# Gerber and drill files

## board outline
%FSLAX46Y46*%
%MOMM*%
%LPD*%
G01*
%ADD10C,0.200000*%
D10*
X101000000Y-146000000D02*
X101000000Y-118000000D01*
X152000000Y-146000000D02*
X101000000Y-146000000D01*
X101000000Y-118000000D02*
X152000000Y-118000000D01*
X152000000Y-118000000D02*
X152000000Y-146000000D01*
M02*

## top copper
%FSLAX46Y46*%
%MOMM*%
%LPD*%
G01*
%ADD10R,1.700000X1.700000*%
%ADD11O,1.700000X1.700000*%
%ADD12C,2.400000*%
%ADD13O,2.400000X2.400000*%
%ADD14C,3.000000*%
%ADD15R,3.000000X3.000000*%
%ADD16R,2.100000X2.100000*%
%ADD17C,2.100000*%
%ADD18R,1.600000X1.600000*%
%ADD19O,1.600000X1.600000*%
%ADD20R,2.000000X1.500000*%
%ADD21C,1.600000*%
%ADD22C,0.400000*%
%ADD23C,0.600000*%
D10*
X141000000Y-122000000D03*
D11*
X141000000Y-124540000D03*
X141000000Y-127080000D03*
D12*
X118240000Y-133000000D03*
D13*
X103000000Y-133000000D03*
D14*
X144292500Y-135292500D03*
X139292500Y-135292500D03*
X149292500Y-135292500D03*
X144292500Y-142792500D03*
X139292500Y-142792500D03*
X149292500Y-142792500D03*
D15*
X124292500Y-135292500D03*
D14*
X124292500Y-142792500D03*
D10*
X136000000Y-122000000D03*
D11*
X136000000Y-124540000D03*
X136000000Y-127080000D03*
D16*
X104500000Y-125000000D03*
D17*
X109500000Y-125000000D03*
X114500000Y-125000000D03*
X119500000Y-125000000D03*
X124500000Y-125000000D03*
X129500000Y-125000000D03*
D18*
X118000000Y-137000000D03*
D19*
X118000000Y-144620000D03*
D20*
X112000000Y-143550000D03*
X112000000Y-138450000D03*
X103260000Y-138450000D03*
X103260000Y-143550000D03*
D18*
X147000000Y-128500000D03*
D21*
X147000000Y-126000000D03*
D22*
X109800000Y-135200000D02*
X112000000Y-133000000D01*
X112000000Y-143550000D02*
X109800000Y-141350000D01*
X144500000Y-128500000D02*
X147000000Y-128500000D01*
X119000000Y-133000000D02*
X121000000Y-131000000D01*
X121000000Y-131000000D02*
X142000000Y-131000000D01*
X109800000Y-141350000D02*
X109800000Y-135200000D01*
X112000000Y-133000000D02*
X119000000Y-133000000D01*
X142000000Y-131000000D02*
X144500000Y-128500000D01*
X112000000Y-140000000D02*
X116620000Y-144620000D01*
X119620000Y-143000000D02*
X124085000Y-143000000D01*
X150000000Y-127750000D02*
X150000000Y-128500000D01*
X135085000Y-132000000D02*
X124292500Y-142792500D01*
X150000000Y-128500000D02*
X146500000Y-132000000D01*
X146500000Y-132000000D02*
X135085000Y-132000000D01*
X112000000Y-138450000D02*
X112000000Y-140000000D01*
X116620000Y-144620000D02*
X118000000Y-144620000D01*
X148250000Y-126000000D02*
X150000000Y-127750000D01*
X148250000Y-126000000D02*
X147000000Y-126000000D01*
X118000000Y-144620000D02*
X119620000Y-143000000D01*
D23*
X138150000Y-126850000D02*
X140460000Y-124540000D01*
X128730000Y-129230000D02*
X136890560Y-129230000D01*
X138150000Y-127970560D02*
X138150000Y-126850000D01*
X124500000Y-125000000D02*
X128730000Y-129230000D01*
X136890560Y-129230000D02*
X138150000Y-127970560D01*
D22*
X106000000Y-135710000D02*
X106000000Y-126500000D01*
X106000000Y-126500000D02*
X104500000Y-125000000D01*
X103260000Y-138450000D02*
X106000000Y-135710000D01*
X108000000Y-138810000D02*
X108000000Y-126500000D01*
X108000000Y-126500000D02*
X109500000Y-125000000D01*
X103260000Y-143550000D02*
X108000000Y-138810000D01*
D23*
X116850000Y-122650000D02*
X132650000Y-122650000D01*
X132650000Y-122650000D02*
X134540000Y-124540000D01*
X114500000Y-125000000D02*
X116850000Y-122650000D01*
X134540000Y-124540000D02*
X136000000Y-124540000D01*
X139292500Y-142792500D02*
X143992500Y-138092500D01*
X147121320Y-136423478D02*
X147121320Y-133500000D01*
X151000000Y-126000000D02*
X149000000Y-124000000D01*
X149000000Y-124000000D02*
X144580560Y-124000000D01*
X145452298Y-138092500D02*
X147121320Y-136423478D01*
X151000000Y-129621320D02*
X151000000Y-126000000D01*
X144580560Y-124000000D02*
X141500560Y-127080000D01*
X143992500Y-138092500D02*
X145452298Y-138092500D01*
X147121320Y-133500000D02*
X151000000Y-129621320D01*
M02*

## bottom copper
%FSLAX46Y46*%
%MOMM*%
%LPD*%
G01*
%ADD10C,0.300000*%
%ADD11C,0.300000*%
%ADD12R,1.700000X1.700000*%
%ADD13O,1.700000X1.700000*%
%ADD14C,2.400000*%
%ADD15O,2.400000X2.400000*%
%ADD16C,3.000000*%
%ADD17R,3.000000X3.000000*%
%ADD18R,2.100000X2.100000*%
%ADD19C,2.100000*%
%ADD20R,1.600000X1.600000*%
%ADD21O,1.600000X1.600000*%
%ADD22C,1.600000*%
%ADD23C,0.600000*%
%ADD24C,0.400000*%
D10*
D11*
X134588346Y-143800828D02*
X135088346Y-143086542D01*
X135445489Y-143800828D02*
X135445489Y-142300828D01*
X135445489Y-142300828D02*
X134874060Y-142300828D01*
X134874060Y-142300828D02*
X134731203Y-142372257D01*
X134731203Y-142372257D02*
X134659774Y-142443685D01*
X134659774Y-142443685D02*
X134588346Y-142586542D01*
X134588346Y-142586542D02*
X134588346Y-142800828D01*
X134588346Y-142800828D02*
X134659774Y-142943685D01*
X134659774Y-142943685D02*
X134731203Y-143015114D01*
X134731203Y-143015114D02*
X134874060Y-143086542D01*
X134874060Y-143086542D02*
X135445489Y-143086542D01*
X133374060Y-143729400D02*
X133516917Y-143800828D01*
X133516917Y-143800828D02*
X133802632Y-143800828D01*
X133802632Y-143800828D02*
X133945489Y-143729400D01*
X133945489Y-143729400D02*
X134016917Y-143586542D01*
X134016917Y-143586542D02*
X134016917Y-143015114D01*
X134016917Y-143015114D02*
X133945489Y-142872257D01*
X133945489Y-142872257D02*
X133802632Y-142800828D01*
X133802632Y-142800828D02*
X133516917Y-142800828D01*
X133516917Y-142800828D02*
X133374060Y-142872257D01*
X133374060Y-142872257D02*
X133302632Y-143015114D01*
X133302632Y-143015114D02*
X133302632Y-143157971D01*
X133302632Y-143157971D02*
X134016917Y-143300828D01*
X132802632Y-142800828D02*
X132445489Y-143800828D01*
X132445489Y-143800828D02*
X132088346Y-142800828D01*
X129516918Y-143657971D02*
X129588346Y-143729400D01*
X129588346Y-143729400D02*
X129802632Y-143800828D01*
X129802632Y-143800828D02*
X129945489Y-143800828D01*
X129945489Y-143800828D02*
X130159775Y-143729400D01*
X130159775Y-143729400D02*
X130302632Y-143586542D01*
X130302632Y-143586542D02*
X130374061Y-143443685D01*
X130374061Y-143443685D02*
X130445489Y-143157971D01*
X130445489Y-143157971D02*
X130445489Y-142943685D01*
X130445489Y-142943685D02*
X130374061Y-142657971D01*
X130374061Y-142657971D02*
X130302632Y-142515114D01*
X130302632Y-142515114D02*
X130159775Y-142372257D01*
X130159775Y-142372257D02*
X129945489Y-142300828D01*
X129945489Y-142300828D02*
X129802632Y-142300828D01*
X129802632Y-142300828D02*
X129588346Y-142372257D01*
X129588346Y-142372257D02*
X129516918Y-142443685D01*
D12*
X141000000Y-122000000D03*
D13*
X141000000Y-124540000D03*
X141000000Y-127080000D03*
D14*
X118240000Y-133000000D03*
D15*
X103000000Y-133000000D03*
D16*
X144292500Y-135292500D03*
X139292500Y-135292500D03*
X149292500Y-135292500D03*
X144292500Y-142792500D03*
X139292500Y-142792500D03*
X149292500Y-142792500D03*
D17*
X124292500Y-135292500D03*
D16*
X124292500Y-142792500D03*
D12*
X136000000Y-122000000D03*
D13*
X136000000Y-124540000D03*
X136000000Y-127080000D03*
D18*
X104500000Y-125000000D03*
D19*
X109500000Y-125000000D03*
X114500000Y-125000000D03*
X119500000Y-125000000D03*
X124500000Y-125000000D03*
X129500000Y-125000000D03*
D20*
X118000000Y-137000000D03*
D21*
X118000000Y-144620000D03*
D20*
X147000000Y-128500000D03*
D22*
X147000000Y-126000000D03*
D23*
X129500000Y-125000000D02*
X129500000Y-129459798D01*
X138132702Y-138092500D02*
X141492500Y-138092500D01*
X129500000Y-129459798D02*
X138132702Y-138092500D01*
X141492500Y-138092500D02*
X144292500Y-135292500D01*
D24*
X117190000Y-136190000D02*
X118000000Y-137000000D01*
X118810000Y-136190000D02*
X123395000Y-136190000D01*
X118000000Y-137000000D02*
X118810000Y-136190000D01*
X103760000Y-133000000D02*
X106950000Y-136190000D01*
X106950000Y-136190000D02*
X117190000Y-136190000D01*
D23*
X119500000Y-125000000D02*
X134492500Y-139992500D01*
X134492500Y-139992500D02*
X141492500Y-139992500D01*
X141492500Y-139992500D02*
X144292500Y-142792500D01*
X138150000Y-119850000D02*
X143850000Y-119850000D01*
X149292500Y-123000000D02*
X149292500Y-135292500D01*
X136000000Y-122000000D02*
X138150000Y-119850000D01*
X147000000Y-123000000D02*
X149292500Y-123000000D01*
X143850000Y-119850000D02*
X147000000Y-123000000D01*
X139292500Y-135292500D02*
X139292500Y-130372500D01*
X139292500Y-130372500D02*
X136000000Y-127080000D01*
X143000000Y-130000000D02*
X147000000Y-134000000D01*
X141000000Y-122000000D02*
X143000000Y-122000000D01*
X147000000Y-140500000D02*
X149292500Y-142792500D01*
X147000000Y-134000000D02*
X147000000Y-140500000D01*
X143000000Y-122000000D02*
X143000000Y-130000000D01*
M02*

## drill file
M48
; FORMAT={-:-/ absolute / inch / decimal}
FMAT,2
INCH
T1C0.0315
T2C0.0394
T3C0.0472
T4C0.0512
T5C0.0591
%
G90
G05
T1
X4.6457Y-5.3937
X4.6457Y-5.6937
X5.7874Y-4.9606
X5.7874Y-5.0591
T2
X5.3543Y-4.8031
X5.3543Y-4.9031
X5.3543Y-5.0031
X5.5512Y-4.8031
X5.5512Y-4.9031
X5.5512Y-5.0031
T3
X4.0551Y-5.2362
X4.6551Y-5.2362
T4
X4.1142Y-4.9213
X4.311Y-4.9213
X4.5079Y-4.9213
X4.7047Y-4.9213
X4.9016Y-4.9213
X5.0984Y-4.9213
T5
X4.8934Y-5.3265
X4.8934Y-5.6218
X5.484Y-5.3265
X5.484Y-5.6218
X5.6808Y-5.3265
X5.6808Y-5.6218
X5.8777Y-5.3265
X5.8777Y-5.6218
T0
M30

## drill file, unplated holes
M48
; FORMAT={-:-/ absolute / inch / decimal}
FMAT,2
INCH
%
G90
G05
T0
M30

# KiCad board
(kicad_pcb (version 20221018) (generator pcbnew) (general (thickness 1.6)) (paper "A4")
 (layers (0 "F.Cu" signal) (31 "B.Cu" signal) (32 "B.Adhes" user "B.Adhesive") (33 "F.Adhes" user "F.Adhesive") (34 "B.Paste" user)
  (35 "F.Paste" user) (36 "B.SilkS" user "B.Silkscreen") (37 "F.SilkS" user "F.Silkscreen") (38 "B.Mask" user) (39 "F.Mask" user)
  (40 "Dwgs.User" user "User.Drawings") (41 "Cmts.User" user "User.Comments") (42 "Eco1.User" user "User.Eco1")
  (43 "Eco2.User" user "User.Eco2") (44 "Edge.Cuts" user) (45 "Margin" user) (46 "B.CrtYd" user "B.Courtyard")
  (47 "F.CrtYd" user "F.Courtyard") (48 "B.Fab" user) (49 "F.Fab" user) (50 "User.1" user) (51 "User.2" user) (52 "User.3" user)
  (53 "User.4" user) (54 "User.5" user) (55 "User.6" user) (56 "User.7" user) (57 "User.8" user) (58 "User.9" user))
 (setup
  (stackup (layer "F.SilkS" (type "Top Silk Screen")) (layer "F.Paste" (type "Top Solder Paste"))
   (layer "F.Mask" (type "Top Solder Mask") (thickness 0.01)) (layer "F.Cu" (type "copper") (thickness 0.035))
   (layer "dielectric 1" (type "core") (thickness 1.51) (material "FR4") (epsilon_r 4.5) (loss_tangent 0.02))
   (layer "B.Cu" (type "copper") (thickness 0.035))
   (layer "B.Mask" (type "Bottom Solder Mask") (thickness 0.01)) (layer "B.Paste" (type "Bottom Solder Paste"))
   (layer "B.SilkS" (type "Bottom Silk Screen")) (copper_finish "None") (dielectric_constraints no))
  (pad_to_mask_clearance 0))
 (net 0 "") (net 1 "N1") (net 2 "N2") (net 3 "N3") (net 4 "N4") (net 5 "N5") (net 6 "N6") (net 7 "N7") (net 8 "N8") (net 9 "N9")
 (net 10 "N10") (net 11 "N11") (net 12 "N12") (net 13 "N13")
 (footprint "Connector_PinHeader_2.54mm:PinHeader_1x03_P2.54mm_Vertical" (layer "F.Cu") (at 141 122)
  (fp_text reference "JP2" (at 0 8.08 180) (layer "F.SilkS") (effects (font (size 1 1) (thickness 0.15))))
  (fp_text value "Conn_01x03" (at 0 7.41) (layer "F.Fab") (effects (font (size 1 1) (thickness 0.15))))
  (pad "1" thru_hole rect (at 0 0) (size 1.7 1.7) (drill 1) (layers "*.Cu" "*.Mask") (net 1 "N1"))
  (pad "2" thru_hole oval (at 0 2.54) (size 1.7 1.7) (drill 1) (layers "*.Cu" "*.Mask") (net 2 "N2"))
  (pad "3" thru_hole oval (at 0 5.08) (size 1.7 1.7) (drill 1) (layers "*.Cu" "*.Mask") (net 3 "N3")))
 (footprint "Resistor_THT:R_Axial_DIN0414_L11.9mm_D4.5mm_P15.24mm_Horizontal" (layer "F.Cu") (at 118.24 133 180)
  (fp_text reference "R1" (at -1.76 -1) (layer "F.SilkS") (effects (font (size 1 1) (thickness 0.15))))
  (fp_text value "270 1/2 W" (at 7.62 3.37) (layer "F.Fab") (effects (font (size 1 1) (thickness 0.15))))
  (pad "1" thru_hole circle (at 0 0 180) (size 2.4 2.4) (drill 1.2) (layers "*.Cu" "*.Mask") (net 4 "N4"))
  (pad "2" thru_hole oval (at 15.24 0 180) (size 2.4 2.4) (drill 1.2) (layers "*.Cu" "*.Mask") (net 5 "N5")))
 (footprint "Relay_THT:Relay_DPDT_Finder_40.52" (layer "F.Cu") (at 124.2925 135.2925)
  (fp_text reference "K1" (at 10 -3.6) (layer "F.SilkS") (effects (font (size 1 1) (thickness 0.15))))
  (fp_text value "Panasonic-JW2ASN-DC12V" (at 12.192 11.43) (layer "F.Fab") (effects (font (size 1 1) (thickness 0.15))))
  (pad "11" thru_hole circle (at 20 0) (size 3 3) (drill 1.5) (layers "*.Cu" "*.Mask") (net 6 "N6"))
  (pad "12" thru_hole circle (at 15 0) (size 3 3) (drill 1.5) (layers "*.Cu" "*.Mask") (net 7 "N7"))
  (pad "14" thru_hole circle (at 25 0) (size 3 3) (drill 1.5) (layers "*.Cu" "*.Mask") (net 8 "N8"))
  (pad "21" thru_hole circle (at 20 7.5) (size 3 3) (drill 1.5) (layers "*.Cu" "*.Mask") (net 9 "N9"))
  (pad "22" thru_hole circle (at 15 7.5) (size 3 3) (drill 1.5) (layers "*.Cu" "*.Mask") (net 3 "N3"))
  (pad "24" thru_hole circle (at 25 7.5) (size 3 3) (drill 1.5) (layers "*.Cu" "*.Mask") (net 1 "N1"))
  (pad "A1" thru_hole rect (at 0 0) (size 3 3) (drill 1.5) (layers "*.Cu" "*.Mask") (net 5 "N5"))
  (pad "A2" thru_hole circle (at 0 7.5) (size 3 3) (drill 1.5) (layers "*.Cu" "*.Mask") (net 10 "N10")))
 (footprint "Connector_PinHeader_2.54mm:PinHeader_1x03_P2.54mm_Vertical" (layer "F.Cu") (at 136 122)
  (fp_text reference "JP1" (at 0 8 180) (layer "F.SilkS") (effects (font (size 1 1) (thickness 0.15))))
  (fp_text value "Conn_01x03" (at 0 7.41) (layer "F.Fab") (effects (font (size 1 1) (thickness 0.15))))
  (pad "1" thru_hole rect (at 0 0) (size 1.7 1.7) (drill 1) (layers "*.Cu" "*.Mask") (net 8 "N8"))
  (pad "2" thru_hole oval (at 0 2.54) (size 1.7 1.7) (drill 1) (layers "*.Cu" "*.Mask") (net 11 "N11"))
  (pad "3" thru_hole oval (at 0 5.08) (size 1.7 1.7) (drill 1) (layers "*.Cu" "*.Mask") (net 7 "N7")))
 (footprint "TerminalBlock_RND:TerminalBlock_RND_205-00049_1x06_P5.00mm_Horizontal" (layer "F.Cu") (at 104.5 125)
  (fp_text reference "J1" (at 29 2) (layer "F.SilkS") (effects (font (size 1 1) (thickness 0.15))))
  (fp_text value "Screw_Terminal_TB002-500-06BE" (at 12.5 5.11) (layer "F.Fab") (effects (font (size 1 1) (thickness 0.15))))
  (pad "1" thru_hole rect (at 0 0) (size 2.1 2.1) (drill 1.3) (layers "*.Cu" "*.Mask") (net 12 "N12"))
  (pad "2" thru_hole circle (at 5 0) (size 2.1 2.1) (drill 1.3) (layers "*.Cu" "*.Mask") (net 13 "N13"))
  (pad "3" thru_hole circle (at 10 0) (size 2.1 2.1) (drill 1.3) (layers "*.Cu" "*.Mask") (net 11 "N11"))
  (pad "4" thru_hole circle (at 15 0) (size 2.1 2.1) (drill 1.3) (layers "*.Cu" "*.Mask") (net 9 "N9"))
  (pad "5" thru_hole circle (at 20 0) (size 2.1 2.1) (drill 1.3) (layers "*.Cu" "*.Mask") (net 2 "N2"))
  (pad "6" thru_hole circle (at 25 0) (size 2.1 2.1) (drill 1.3) (layers "*.Cu" "*.Mask") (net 6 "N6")))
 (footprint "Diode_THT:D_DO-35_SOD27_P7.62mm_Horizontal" (layer "F.Cu") (at 118 137 -90)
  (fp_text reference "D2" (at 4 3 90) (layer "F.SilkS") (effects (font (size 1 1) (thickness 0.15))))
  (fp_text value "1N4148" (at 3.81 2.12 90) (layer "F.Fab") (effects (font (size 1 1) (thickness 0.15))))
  (pad "1" thru_hole rect (at 0 0 270) (size 1.6 1.6) (drill 0.8) (layers "*.Cu" "*.Mask") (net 5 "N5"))
  (pad "2" thru_hole oval (at 7.62 0 270) (size 1.6 1.6) (drill 0.8) (layers "*.Cu" "*.Mask") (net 10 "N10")))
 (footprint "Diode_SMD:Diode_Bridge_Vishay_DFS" (layer "F.Cu") (at 107.63 141 180)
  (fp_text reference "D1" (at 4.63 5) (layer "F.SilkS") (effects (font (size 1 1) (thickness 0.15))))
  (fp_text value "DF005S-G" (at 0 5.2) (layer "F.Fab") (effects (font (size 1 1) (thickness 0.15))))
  (pad "1" smd rect (at -4.37 -2.55 180) (size 2 1.5) (layers "F.Cu" "F.Paste" "F.Mask") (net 4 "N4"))
  (pad "2" smd rect (at -4.37 2.55 180) (size 2 1.5) (layers "F.Cu" "F.Paste" "F.Mask") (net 10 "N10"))
  (pad "3" smd rect (at 4.37 2.55 180) (size 2 1.5) (layers "F.Cu" "F.Paste" "F.Mask") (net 12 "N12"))
  (pad "4" smd rect (at 4.37 -2.55 180) (size 2 1.5) (layers "F.Cu" "F.Paste" "F.Mask") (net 13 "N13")))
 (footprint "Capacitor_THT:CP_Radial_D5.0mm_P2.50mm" (layer "F.Cu") (at 147 128.5 90)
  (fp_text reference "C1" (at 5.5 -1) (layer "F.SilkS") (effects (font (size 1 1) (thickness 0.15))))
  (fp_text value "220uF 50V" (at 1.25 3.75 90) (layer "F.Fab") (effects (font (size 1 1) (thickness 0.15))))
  (pad "1" thru_hole rect (at 0 0 90) (size 1.6 1.6) (drill 0.8) (layers "*.Cu" "*.Mask") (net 4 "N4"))
  (pad "2" thru_hole circle (at 2.5 0 90) (size 1.6 1.6) (drill 0.8) (layers "*.Cu" "*.Mask") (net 10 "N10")))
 (gr_line (start 101 146) (end 101 118) (stroke (width 0.2) (type default)) (layer "Edge.Cuts"))
 (gr_line (start 152 146) (end 101 146) (stroke (width 0.2) (type default)) (layer "Edge.Cuts"))
 (gr_line (start 101 118) (end 152 118) (stroke (width 0.2) (type default)) (layer "Edge.Cuts"))
 (gr_line (start 152 118) (end 152 146) (stroke (width 0.2) (type default)) (layer "Edge.Cuts"))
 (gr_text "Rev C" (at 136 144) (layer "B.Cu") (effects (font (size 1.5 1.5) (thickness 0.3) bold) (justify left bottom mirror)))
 (segment (start 109.8 135.2) (end 112 133) (width 0.4) (layer "F.Cu") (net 4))
 (segment (start 112 143.55) (end 109.8 141.35) (width 0.4) (layer "F.Cu") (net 4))
 (segment (start 144.5 128.5) (end 147 128.5) (width 0.4) (layer "F.Cu") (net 4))
 (segment (start 119 133) (end 121 131) (width 0.4) (layer "F.Cu") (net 4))
 (segment (start 121 131) (end 142 131) (width 0.4) (layer "F.Cu") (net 4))
 (segment (start 109.8 141.35) (end 109.8 135.2) (width 0.4) (layer "F.Cu") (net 4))
 (segment (start 112 133) (end 119 133) (width 0.4) (layer "F.Cu") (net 4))
 (segment (start 142 131) (end 144.5 128.5) (width 0.4) (layer "F.Cu") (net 4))
 (segment (start 112 140) (end 116.62 144.62) (width 0.4) (layer "F.Cu") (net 10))
 (segment (start 119.62 143) (end 124.085 143) (width 0.4) (layer "F.Cu") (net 10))
 (segment (start 150 127.75) (end 150 128.5) (width 0.4) (layer "F.Cu") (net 10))
 (segment (start 135.085 132) (end 124.2925 142.7925) (width 0.4) (layer "F.Cu") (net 10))
 (segment (start 150 128.5) (end 146.5 132) (width 0.4) (layer "F.Cu") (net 10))
 (segment (start 146.5 132) (end 135.085 132) (width 0.4) (layer "F.Cu") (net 10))
 (segment (start 112 138.45) (end 112 140) (width 0.4) (layer "F.Cu") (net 10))
 (segment (start 116.62 144.62) (end 118 144.62) (width 0.4) (layer "F.Cu") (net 10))
 (segment (start 148.25 126) (end 150 127.75) (width 0.4) (layer "F.Cu") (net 10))
 (segment (start 148.25 126) (end 147 126) (width 0.4) (layer "F.Cu") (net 10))
 (segment (start 118 144.62) (end 119.62 143) (width 0.4) (layer "F.Cu") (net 10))
 (segment (start 138.15 126.85) (end 140.46 124.54) (width 0.6) (layer "F.Cu") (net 2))
 (segment (start 128.73 129.23) (end 136.89056 129.23) (width 0.6) (layer "F.Cu") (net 2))
 (segment (start 138.15 127.97056) (end 138.15 126.85) (width 0.6) (layer "F.Cu") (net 2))
 (segment (start 124.5 125) (end 128.73 129.23) (width 0.6) (layer "F.Cu") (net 2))
 (segment (start 136.89056 129.23) (end 138.15 127.97056) (width 0.6) (layer "F.Cu") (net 2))
 (segment (start 129.5 125) (end 129.5 129.459798) (width 0.6) (layer "B.Cu") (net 6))
 (segment (start 138.132702 138.0925) (end 141.4925 138.0925) (width 0.6) (layer "B.Cu") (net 6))
 (segment (start 129.5 129.459798) (end 138.132702 138.0925) (width 0.6) (layer "B.Cu") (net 6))
 (segment (start 141.4925 138.0925) (end 144.2925 135.2925) (width 0.6) (layer "B.Cu") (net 6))
 (segment (start 117.19 136.19) (end 118 137) (width 0.4) (layer "B.Cu") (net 5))
 (segment (start 118.81 136.19) (end 123.395 136.19) (width 0.4) (layer "B.Cu") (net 5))
 (segment (start 118 137) (end 118.81 136.19) (width 0.4) (layer "B.Cu") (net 5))
 (segment (start 103.76 133) (end 106.95 136.19) (width 0.4) (layer "B.Cu") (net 5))
 (segment (start 106.95 136.19) (end 117.19 136.19) (width 0.4) (layer "B.Cu") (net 5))
 (segment (start 106 135.71) (end 106 126.5) (width 0.4) (layer "F.Cu") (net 12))
 (segment (start 106 126.5) (end 104.5 125) (width 0.4) (layer "F.Cu") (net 12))
 (segment (start 103.26 138.45) (end 106 135.71) (width 0.4) (layer "F.Cu") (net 12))
 (segment (start 108 138.81) (end 108 126.5) (width 0.4) (layer "F.Cu") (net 13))
 (segment (start 108 126.5) (end 109.5 125) (width 0.4) (layer "F.Cu") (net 13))
 (segment (start 103.26 143.55) (end 108 138.81) (width 0.4) (layer "F.Cu") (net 13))
 (segment (start 116.85 122.65) (end 132.65 122.65) (width 0.6) (layer "F.Cu") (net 11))
 (segment (start 132.65 122.65) (end 134.54 124.54) (width 0.6) (layer "F.Cu") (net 11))
 (segment (start 114.5 125) (end 116.85 122.65) (width 0.6) (layer "F.Cu") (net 11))
 (segment (start 134.54 124.54) (end 136 124.54) (width 0.6) (layer "F.Cu") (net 11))
 (segment (start 119.5 125) (end 134.4925 139.9925) (width 0.6) (layer "B.Cu") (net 9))
 (segment (start 134.4925 139.9925) (end 141.4925 139.9925) (width 0.6) (layer "B.Cu") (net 9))
 (segment (start 141.4925 139.9925) (end 144.2925 142.7925) (width 0.6) (layer "B.Cu") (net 9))
 (segment (start 138.15 119.85) (end 143.85 119.85) (width 0.6) (layer "B.Cu") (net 8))
 (segment (start 149.2925 123) (end 149.2925 135.2925) (width 0.6) (layer "B.Cu") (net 8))
 (segment (start 136 122) (end 138.15 119.85) (width 0.6) (layer "B.Cu") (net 8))
 (segment (start 147 123) (end 149.2925 123) (width 0.6) (layer "B.Cu") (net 8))
 (segment (start 143.85 119.85) (end 147 123) (width 0.6) (layer "B.Cu") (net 8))
 (segment (start 139.2925 135.2925) (end 139.2925 130.3725) (width 0.6) (layer "B.Cu") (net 7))
 (segment (start 139.2925 130.3725) (end 136 127.08) (width 0.6) (layer "B.Cu") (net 7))
 (segment (start 143 130) (end 147 134) (width 0.6) (layer "B.Cu") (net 1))
 (segment (start 141 122) (end 143 122) (width 0.6) (layer "B.Cu") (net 1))
 (segment (start 147 140.5) (end 149.2925 142.7925) (width 0.6) (layer "B.Cu") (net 1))
 (segment (start 147 134) (end 147 140.5) (width 0.6) (layer "B.Cu") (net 1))
 (segment (start 143 122) (end 143 130) (width 0.6) (layer "B.Cu") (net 1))
 (segment (start 139.2925 142.7925) (end 143.9925 138.0925) (width 0.6) (layer "F.Cu") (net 3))
 (segment (start 147.12132 136.423478) (end 147.12132 133.5) (width 0.6) (layer "F.Cu") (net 3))
 (segment (start 151 126) (end 149 124) (width 0.6) (layer "F.Cu") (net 3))
 (segment (start 149 124) (end 144.58056 124) (width 0.6) (layer "F.Cu") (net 3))
 (segment (start 145.452298 138.0925) (end 147.12132 136.423478) (width 0.6) (layer "F.Cu") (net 3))
 (segment (start 151 129.62132) (end 151 126) (width 0.6) (layer "F.Cu") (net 3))
 (segment (start 144.58056 124) (end 141.50056 127.08) (width 0.6) (layer "F.Cu") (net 3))
 (segment (start 143.9925 138.0925) (end 145.452298 138.0925) (width 0.6) (layer "F.Cu") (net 3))
 (segment (start 147.12132 133.5) (end 151 129.62132) (width 0.6) (layer "F.Cu") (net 3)))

